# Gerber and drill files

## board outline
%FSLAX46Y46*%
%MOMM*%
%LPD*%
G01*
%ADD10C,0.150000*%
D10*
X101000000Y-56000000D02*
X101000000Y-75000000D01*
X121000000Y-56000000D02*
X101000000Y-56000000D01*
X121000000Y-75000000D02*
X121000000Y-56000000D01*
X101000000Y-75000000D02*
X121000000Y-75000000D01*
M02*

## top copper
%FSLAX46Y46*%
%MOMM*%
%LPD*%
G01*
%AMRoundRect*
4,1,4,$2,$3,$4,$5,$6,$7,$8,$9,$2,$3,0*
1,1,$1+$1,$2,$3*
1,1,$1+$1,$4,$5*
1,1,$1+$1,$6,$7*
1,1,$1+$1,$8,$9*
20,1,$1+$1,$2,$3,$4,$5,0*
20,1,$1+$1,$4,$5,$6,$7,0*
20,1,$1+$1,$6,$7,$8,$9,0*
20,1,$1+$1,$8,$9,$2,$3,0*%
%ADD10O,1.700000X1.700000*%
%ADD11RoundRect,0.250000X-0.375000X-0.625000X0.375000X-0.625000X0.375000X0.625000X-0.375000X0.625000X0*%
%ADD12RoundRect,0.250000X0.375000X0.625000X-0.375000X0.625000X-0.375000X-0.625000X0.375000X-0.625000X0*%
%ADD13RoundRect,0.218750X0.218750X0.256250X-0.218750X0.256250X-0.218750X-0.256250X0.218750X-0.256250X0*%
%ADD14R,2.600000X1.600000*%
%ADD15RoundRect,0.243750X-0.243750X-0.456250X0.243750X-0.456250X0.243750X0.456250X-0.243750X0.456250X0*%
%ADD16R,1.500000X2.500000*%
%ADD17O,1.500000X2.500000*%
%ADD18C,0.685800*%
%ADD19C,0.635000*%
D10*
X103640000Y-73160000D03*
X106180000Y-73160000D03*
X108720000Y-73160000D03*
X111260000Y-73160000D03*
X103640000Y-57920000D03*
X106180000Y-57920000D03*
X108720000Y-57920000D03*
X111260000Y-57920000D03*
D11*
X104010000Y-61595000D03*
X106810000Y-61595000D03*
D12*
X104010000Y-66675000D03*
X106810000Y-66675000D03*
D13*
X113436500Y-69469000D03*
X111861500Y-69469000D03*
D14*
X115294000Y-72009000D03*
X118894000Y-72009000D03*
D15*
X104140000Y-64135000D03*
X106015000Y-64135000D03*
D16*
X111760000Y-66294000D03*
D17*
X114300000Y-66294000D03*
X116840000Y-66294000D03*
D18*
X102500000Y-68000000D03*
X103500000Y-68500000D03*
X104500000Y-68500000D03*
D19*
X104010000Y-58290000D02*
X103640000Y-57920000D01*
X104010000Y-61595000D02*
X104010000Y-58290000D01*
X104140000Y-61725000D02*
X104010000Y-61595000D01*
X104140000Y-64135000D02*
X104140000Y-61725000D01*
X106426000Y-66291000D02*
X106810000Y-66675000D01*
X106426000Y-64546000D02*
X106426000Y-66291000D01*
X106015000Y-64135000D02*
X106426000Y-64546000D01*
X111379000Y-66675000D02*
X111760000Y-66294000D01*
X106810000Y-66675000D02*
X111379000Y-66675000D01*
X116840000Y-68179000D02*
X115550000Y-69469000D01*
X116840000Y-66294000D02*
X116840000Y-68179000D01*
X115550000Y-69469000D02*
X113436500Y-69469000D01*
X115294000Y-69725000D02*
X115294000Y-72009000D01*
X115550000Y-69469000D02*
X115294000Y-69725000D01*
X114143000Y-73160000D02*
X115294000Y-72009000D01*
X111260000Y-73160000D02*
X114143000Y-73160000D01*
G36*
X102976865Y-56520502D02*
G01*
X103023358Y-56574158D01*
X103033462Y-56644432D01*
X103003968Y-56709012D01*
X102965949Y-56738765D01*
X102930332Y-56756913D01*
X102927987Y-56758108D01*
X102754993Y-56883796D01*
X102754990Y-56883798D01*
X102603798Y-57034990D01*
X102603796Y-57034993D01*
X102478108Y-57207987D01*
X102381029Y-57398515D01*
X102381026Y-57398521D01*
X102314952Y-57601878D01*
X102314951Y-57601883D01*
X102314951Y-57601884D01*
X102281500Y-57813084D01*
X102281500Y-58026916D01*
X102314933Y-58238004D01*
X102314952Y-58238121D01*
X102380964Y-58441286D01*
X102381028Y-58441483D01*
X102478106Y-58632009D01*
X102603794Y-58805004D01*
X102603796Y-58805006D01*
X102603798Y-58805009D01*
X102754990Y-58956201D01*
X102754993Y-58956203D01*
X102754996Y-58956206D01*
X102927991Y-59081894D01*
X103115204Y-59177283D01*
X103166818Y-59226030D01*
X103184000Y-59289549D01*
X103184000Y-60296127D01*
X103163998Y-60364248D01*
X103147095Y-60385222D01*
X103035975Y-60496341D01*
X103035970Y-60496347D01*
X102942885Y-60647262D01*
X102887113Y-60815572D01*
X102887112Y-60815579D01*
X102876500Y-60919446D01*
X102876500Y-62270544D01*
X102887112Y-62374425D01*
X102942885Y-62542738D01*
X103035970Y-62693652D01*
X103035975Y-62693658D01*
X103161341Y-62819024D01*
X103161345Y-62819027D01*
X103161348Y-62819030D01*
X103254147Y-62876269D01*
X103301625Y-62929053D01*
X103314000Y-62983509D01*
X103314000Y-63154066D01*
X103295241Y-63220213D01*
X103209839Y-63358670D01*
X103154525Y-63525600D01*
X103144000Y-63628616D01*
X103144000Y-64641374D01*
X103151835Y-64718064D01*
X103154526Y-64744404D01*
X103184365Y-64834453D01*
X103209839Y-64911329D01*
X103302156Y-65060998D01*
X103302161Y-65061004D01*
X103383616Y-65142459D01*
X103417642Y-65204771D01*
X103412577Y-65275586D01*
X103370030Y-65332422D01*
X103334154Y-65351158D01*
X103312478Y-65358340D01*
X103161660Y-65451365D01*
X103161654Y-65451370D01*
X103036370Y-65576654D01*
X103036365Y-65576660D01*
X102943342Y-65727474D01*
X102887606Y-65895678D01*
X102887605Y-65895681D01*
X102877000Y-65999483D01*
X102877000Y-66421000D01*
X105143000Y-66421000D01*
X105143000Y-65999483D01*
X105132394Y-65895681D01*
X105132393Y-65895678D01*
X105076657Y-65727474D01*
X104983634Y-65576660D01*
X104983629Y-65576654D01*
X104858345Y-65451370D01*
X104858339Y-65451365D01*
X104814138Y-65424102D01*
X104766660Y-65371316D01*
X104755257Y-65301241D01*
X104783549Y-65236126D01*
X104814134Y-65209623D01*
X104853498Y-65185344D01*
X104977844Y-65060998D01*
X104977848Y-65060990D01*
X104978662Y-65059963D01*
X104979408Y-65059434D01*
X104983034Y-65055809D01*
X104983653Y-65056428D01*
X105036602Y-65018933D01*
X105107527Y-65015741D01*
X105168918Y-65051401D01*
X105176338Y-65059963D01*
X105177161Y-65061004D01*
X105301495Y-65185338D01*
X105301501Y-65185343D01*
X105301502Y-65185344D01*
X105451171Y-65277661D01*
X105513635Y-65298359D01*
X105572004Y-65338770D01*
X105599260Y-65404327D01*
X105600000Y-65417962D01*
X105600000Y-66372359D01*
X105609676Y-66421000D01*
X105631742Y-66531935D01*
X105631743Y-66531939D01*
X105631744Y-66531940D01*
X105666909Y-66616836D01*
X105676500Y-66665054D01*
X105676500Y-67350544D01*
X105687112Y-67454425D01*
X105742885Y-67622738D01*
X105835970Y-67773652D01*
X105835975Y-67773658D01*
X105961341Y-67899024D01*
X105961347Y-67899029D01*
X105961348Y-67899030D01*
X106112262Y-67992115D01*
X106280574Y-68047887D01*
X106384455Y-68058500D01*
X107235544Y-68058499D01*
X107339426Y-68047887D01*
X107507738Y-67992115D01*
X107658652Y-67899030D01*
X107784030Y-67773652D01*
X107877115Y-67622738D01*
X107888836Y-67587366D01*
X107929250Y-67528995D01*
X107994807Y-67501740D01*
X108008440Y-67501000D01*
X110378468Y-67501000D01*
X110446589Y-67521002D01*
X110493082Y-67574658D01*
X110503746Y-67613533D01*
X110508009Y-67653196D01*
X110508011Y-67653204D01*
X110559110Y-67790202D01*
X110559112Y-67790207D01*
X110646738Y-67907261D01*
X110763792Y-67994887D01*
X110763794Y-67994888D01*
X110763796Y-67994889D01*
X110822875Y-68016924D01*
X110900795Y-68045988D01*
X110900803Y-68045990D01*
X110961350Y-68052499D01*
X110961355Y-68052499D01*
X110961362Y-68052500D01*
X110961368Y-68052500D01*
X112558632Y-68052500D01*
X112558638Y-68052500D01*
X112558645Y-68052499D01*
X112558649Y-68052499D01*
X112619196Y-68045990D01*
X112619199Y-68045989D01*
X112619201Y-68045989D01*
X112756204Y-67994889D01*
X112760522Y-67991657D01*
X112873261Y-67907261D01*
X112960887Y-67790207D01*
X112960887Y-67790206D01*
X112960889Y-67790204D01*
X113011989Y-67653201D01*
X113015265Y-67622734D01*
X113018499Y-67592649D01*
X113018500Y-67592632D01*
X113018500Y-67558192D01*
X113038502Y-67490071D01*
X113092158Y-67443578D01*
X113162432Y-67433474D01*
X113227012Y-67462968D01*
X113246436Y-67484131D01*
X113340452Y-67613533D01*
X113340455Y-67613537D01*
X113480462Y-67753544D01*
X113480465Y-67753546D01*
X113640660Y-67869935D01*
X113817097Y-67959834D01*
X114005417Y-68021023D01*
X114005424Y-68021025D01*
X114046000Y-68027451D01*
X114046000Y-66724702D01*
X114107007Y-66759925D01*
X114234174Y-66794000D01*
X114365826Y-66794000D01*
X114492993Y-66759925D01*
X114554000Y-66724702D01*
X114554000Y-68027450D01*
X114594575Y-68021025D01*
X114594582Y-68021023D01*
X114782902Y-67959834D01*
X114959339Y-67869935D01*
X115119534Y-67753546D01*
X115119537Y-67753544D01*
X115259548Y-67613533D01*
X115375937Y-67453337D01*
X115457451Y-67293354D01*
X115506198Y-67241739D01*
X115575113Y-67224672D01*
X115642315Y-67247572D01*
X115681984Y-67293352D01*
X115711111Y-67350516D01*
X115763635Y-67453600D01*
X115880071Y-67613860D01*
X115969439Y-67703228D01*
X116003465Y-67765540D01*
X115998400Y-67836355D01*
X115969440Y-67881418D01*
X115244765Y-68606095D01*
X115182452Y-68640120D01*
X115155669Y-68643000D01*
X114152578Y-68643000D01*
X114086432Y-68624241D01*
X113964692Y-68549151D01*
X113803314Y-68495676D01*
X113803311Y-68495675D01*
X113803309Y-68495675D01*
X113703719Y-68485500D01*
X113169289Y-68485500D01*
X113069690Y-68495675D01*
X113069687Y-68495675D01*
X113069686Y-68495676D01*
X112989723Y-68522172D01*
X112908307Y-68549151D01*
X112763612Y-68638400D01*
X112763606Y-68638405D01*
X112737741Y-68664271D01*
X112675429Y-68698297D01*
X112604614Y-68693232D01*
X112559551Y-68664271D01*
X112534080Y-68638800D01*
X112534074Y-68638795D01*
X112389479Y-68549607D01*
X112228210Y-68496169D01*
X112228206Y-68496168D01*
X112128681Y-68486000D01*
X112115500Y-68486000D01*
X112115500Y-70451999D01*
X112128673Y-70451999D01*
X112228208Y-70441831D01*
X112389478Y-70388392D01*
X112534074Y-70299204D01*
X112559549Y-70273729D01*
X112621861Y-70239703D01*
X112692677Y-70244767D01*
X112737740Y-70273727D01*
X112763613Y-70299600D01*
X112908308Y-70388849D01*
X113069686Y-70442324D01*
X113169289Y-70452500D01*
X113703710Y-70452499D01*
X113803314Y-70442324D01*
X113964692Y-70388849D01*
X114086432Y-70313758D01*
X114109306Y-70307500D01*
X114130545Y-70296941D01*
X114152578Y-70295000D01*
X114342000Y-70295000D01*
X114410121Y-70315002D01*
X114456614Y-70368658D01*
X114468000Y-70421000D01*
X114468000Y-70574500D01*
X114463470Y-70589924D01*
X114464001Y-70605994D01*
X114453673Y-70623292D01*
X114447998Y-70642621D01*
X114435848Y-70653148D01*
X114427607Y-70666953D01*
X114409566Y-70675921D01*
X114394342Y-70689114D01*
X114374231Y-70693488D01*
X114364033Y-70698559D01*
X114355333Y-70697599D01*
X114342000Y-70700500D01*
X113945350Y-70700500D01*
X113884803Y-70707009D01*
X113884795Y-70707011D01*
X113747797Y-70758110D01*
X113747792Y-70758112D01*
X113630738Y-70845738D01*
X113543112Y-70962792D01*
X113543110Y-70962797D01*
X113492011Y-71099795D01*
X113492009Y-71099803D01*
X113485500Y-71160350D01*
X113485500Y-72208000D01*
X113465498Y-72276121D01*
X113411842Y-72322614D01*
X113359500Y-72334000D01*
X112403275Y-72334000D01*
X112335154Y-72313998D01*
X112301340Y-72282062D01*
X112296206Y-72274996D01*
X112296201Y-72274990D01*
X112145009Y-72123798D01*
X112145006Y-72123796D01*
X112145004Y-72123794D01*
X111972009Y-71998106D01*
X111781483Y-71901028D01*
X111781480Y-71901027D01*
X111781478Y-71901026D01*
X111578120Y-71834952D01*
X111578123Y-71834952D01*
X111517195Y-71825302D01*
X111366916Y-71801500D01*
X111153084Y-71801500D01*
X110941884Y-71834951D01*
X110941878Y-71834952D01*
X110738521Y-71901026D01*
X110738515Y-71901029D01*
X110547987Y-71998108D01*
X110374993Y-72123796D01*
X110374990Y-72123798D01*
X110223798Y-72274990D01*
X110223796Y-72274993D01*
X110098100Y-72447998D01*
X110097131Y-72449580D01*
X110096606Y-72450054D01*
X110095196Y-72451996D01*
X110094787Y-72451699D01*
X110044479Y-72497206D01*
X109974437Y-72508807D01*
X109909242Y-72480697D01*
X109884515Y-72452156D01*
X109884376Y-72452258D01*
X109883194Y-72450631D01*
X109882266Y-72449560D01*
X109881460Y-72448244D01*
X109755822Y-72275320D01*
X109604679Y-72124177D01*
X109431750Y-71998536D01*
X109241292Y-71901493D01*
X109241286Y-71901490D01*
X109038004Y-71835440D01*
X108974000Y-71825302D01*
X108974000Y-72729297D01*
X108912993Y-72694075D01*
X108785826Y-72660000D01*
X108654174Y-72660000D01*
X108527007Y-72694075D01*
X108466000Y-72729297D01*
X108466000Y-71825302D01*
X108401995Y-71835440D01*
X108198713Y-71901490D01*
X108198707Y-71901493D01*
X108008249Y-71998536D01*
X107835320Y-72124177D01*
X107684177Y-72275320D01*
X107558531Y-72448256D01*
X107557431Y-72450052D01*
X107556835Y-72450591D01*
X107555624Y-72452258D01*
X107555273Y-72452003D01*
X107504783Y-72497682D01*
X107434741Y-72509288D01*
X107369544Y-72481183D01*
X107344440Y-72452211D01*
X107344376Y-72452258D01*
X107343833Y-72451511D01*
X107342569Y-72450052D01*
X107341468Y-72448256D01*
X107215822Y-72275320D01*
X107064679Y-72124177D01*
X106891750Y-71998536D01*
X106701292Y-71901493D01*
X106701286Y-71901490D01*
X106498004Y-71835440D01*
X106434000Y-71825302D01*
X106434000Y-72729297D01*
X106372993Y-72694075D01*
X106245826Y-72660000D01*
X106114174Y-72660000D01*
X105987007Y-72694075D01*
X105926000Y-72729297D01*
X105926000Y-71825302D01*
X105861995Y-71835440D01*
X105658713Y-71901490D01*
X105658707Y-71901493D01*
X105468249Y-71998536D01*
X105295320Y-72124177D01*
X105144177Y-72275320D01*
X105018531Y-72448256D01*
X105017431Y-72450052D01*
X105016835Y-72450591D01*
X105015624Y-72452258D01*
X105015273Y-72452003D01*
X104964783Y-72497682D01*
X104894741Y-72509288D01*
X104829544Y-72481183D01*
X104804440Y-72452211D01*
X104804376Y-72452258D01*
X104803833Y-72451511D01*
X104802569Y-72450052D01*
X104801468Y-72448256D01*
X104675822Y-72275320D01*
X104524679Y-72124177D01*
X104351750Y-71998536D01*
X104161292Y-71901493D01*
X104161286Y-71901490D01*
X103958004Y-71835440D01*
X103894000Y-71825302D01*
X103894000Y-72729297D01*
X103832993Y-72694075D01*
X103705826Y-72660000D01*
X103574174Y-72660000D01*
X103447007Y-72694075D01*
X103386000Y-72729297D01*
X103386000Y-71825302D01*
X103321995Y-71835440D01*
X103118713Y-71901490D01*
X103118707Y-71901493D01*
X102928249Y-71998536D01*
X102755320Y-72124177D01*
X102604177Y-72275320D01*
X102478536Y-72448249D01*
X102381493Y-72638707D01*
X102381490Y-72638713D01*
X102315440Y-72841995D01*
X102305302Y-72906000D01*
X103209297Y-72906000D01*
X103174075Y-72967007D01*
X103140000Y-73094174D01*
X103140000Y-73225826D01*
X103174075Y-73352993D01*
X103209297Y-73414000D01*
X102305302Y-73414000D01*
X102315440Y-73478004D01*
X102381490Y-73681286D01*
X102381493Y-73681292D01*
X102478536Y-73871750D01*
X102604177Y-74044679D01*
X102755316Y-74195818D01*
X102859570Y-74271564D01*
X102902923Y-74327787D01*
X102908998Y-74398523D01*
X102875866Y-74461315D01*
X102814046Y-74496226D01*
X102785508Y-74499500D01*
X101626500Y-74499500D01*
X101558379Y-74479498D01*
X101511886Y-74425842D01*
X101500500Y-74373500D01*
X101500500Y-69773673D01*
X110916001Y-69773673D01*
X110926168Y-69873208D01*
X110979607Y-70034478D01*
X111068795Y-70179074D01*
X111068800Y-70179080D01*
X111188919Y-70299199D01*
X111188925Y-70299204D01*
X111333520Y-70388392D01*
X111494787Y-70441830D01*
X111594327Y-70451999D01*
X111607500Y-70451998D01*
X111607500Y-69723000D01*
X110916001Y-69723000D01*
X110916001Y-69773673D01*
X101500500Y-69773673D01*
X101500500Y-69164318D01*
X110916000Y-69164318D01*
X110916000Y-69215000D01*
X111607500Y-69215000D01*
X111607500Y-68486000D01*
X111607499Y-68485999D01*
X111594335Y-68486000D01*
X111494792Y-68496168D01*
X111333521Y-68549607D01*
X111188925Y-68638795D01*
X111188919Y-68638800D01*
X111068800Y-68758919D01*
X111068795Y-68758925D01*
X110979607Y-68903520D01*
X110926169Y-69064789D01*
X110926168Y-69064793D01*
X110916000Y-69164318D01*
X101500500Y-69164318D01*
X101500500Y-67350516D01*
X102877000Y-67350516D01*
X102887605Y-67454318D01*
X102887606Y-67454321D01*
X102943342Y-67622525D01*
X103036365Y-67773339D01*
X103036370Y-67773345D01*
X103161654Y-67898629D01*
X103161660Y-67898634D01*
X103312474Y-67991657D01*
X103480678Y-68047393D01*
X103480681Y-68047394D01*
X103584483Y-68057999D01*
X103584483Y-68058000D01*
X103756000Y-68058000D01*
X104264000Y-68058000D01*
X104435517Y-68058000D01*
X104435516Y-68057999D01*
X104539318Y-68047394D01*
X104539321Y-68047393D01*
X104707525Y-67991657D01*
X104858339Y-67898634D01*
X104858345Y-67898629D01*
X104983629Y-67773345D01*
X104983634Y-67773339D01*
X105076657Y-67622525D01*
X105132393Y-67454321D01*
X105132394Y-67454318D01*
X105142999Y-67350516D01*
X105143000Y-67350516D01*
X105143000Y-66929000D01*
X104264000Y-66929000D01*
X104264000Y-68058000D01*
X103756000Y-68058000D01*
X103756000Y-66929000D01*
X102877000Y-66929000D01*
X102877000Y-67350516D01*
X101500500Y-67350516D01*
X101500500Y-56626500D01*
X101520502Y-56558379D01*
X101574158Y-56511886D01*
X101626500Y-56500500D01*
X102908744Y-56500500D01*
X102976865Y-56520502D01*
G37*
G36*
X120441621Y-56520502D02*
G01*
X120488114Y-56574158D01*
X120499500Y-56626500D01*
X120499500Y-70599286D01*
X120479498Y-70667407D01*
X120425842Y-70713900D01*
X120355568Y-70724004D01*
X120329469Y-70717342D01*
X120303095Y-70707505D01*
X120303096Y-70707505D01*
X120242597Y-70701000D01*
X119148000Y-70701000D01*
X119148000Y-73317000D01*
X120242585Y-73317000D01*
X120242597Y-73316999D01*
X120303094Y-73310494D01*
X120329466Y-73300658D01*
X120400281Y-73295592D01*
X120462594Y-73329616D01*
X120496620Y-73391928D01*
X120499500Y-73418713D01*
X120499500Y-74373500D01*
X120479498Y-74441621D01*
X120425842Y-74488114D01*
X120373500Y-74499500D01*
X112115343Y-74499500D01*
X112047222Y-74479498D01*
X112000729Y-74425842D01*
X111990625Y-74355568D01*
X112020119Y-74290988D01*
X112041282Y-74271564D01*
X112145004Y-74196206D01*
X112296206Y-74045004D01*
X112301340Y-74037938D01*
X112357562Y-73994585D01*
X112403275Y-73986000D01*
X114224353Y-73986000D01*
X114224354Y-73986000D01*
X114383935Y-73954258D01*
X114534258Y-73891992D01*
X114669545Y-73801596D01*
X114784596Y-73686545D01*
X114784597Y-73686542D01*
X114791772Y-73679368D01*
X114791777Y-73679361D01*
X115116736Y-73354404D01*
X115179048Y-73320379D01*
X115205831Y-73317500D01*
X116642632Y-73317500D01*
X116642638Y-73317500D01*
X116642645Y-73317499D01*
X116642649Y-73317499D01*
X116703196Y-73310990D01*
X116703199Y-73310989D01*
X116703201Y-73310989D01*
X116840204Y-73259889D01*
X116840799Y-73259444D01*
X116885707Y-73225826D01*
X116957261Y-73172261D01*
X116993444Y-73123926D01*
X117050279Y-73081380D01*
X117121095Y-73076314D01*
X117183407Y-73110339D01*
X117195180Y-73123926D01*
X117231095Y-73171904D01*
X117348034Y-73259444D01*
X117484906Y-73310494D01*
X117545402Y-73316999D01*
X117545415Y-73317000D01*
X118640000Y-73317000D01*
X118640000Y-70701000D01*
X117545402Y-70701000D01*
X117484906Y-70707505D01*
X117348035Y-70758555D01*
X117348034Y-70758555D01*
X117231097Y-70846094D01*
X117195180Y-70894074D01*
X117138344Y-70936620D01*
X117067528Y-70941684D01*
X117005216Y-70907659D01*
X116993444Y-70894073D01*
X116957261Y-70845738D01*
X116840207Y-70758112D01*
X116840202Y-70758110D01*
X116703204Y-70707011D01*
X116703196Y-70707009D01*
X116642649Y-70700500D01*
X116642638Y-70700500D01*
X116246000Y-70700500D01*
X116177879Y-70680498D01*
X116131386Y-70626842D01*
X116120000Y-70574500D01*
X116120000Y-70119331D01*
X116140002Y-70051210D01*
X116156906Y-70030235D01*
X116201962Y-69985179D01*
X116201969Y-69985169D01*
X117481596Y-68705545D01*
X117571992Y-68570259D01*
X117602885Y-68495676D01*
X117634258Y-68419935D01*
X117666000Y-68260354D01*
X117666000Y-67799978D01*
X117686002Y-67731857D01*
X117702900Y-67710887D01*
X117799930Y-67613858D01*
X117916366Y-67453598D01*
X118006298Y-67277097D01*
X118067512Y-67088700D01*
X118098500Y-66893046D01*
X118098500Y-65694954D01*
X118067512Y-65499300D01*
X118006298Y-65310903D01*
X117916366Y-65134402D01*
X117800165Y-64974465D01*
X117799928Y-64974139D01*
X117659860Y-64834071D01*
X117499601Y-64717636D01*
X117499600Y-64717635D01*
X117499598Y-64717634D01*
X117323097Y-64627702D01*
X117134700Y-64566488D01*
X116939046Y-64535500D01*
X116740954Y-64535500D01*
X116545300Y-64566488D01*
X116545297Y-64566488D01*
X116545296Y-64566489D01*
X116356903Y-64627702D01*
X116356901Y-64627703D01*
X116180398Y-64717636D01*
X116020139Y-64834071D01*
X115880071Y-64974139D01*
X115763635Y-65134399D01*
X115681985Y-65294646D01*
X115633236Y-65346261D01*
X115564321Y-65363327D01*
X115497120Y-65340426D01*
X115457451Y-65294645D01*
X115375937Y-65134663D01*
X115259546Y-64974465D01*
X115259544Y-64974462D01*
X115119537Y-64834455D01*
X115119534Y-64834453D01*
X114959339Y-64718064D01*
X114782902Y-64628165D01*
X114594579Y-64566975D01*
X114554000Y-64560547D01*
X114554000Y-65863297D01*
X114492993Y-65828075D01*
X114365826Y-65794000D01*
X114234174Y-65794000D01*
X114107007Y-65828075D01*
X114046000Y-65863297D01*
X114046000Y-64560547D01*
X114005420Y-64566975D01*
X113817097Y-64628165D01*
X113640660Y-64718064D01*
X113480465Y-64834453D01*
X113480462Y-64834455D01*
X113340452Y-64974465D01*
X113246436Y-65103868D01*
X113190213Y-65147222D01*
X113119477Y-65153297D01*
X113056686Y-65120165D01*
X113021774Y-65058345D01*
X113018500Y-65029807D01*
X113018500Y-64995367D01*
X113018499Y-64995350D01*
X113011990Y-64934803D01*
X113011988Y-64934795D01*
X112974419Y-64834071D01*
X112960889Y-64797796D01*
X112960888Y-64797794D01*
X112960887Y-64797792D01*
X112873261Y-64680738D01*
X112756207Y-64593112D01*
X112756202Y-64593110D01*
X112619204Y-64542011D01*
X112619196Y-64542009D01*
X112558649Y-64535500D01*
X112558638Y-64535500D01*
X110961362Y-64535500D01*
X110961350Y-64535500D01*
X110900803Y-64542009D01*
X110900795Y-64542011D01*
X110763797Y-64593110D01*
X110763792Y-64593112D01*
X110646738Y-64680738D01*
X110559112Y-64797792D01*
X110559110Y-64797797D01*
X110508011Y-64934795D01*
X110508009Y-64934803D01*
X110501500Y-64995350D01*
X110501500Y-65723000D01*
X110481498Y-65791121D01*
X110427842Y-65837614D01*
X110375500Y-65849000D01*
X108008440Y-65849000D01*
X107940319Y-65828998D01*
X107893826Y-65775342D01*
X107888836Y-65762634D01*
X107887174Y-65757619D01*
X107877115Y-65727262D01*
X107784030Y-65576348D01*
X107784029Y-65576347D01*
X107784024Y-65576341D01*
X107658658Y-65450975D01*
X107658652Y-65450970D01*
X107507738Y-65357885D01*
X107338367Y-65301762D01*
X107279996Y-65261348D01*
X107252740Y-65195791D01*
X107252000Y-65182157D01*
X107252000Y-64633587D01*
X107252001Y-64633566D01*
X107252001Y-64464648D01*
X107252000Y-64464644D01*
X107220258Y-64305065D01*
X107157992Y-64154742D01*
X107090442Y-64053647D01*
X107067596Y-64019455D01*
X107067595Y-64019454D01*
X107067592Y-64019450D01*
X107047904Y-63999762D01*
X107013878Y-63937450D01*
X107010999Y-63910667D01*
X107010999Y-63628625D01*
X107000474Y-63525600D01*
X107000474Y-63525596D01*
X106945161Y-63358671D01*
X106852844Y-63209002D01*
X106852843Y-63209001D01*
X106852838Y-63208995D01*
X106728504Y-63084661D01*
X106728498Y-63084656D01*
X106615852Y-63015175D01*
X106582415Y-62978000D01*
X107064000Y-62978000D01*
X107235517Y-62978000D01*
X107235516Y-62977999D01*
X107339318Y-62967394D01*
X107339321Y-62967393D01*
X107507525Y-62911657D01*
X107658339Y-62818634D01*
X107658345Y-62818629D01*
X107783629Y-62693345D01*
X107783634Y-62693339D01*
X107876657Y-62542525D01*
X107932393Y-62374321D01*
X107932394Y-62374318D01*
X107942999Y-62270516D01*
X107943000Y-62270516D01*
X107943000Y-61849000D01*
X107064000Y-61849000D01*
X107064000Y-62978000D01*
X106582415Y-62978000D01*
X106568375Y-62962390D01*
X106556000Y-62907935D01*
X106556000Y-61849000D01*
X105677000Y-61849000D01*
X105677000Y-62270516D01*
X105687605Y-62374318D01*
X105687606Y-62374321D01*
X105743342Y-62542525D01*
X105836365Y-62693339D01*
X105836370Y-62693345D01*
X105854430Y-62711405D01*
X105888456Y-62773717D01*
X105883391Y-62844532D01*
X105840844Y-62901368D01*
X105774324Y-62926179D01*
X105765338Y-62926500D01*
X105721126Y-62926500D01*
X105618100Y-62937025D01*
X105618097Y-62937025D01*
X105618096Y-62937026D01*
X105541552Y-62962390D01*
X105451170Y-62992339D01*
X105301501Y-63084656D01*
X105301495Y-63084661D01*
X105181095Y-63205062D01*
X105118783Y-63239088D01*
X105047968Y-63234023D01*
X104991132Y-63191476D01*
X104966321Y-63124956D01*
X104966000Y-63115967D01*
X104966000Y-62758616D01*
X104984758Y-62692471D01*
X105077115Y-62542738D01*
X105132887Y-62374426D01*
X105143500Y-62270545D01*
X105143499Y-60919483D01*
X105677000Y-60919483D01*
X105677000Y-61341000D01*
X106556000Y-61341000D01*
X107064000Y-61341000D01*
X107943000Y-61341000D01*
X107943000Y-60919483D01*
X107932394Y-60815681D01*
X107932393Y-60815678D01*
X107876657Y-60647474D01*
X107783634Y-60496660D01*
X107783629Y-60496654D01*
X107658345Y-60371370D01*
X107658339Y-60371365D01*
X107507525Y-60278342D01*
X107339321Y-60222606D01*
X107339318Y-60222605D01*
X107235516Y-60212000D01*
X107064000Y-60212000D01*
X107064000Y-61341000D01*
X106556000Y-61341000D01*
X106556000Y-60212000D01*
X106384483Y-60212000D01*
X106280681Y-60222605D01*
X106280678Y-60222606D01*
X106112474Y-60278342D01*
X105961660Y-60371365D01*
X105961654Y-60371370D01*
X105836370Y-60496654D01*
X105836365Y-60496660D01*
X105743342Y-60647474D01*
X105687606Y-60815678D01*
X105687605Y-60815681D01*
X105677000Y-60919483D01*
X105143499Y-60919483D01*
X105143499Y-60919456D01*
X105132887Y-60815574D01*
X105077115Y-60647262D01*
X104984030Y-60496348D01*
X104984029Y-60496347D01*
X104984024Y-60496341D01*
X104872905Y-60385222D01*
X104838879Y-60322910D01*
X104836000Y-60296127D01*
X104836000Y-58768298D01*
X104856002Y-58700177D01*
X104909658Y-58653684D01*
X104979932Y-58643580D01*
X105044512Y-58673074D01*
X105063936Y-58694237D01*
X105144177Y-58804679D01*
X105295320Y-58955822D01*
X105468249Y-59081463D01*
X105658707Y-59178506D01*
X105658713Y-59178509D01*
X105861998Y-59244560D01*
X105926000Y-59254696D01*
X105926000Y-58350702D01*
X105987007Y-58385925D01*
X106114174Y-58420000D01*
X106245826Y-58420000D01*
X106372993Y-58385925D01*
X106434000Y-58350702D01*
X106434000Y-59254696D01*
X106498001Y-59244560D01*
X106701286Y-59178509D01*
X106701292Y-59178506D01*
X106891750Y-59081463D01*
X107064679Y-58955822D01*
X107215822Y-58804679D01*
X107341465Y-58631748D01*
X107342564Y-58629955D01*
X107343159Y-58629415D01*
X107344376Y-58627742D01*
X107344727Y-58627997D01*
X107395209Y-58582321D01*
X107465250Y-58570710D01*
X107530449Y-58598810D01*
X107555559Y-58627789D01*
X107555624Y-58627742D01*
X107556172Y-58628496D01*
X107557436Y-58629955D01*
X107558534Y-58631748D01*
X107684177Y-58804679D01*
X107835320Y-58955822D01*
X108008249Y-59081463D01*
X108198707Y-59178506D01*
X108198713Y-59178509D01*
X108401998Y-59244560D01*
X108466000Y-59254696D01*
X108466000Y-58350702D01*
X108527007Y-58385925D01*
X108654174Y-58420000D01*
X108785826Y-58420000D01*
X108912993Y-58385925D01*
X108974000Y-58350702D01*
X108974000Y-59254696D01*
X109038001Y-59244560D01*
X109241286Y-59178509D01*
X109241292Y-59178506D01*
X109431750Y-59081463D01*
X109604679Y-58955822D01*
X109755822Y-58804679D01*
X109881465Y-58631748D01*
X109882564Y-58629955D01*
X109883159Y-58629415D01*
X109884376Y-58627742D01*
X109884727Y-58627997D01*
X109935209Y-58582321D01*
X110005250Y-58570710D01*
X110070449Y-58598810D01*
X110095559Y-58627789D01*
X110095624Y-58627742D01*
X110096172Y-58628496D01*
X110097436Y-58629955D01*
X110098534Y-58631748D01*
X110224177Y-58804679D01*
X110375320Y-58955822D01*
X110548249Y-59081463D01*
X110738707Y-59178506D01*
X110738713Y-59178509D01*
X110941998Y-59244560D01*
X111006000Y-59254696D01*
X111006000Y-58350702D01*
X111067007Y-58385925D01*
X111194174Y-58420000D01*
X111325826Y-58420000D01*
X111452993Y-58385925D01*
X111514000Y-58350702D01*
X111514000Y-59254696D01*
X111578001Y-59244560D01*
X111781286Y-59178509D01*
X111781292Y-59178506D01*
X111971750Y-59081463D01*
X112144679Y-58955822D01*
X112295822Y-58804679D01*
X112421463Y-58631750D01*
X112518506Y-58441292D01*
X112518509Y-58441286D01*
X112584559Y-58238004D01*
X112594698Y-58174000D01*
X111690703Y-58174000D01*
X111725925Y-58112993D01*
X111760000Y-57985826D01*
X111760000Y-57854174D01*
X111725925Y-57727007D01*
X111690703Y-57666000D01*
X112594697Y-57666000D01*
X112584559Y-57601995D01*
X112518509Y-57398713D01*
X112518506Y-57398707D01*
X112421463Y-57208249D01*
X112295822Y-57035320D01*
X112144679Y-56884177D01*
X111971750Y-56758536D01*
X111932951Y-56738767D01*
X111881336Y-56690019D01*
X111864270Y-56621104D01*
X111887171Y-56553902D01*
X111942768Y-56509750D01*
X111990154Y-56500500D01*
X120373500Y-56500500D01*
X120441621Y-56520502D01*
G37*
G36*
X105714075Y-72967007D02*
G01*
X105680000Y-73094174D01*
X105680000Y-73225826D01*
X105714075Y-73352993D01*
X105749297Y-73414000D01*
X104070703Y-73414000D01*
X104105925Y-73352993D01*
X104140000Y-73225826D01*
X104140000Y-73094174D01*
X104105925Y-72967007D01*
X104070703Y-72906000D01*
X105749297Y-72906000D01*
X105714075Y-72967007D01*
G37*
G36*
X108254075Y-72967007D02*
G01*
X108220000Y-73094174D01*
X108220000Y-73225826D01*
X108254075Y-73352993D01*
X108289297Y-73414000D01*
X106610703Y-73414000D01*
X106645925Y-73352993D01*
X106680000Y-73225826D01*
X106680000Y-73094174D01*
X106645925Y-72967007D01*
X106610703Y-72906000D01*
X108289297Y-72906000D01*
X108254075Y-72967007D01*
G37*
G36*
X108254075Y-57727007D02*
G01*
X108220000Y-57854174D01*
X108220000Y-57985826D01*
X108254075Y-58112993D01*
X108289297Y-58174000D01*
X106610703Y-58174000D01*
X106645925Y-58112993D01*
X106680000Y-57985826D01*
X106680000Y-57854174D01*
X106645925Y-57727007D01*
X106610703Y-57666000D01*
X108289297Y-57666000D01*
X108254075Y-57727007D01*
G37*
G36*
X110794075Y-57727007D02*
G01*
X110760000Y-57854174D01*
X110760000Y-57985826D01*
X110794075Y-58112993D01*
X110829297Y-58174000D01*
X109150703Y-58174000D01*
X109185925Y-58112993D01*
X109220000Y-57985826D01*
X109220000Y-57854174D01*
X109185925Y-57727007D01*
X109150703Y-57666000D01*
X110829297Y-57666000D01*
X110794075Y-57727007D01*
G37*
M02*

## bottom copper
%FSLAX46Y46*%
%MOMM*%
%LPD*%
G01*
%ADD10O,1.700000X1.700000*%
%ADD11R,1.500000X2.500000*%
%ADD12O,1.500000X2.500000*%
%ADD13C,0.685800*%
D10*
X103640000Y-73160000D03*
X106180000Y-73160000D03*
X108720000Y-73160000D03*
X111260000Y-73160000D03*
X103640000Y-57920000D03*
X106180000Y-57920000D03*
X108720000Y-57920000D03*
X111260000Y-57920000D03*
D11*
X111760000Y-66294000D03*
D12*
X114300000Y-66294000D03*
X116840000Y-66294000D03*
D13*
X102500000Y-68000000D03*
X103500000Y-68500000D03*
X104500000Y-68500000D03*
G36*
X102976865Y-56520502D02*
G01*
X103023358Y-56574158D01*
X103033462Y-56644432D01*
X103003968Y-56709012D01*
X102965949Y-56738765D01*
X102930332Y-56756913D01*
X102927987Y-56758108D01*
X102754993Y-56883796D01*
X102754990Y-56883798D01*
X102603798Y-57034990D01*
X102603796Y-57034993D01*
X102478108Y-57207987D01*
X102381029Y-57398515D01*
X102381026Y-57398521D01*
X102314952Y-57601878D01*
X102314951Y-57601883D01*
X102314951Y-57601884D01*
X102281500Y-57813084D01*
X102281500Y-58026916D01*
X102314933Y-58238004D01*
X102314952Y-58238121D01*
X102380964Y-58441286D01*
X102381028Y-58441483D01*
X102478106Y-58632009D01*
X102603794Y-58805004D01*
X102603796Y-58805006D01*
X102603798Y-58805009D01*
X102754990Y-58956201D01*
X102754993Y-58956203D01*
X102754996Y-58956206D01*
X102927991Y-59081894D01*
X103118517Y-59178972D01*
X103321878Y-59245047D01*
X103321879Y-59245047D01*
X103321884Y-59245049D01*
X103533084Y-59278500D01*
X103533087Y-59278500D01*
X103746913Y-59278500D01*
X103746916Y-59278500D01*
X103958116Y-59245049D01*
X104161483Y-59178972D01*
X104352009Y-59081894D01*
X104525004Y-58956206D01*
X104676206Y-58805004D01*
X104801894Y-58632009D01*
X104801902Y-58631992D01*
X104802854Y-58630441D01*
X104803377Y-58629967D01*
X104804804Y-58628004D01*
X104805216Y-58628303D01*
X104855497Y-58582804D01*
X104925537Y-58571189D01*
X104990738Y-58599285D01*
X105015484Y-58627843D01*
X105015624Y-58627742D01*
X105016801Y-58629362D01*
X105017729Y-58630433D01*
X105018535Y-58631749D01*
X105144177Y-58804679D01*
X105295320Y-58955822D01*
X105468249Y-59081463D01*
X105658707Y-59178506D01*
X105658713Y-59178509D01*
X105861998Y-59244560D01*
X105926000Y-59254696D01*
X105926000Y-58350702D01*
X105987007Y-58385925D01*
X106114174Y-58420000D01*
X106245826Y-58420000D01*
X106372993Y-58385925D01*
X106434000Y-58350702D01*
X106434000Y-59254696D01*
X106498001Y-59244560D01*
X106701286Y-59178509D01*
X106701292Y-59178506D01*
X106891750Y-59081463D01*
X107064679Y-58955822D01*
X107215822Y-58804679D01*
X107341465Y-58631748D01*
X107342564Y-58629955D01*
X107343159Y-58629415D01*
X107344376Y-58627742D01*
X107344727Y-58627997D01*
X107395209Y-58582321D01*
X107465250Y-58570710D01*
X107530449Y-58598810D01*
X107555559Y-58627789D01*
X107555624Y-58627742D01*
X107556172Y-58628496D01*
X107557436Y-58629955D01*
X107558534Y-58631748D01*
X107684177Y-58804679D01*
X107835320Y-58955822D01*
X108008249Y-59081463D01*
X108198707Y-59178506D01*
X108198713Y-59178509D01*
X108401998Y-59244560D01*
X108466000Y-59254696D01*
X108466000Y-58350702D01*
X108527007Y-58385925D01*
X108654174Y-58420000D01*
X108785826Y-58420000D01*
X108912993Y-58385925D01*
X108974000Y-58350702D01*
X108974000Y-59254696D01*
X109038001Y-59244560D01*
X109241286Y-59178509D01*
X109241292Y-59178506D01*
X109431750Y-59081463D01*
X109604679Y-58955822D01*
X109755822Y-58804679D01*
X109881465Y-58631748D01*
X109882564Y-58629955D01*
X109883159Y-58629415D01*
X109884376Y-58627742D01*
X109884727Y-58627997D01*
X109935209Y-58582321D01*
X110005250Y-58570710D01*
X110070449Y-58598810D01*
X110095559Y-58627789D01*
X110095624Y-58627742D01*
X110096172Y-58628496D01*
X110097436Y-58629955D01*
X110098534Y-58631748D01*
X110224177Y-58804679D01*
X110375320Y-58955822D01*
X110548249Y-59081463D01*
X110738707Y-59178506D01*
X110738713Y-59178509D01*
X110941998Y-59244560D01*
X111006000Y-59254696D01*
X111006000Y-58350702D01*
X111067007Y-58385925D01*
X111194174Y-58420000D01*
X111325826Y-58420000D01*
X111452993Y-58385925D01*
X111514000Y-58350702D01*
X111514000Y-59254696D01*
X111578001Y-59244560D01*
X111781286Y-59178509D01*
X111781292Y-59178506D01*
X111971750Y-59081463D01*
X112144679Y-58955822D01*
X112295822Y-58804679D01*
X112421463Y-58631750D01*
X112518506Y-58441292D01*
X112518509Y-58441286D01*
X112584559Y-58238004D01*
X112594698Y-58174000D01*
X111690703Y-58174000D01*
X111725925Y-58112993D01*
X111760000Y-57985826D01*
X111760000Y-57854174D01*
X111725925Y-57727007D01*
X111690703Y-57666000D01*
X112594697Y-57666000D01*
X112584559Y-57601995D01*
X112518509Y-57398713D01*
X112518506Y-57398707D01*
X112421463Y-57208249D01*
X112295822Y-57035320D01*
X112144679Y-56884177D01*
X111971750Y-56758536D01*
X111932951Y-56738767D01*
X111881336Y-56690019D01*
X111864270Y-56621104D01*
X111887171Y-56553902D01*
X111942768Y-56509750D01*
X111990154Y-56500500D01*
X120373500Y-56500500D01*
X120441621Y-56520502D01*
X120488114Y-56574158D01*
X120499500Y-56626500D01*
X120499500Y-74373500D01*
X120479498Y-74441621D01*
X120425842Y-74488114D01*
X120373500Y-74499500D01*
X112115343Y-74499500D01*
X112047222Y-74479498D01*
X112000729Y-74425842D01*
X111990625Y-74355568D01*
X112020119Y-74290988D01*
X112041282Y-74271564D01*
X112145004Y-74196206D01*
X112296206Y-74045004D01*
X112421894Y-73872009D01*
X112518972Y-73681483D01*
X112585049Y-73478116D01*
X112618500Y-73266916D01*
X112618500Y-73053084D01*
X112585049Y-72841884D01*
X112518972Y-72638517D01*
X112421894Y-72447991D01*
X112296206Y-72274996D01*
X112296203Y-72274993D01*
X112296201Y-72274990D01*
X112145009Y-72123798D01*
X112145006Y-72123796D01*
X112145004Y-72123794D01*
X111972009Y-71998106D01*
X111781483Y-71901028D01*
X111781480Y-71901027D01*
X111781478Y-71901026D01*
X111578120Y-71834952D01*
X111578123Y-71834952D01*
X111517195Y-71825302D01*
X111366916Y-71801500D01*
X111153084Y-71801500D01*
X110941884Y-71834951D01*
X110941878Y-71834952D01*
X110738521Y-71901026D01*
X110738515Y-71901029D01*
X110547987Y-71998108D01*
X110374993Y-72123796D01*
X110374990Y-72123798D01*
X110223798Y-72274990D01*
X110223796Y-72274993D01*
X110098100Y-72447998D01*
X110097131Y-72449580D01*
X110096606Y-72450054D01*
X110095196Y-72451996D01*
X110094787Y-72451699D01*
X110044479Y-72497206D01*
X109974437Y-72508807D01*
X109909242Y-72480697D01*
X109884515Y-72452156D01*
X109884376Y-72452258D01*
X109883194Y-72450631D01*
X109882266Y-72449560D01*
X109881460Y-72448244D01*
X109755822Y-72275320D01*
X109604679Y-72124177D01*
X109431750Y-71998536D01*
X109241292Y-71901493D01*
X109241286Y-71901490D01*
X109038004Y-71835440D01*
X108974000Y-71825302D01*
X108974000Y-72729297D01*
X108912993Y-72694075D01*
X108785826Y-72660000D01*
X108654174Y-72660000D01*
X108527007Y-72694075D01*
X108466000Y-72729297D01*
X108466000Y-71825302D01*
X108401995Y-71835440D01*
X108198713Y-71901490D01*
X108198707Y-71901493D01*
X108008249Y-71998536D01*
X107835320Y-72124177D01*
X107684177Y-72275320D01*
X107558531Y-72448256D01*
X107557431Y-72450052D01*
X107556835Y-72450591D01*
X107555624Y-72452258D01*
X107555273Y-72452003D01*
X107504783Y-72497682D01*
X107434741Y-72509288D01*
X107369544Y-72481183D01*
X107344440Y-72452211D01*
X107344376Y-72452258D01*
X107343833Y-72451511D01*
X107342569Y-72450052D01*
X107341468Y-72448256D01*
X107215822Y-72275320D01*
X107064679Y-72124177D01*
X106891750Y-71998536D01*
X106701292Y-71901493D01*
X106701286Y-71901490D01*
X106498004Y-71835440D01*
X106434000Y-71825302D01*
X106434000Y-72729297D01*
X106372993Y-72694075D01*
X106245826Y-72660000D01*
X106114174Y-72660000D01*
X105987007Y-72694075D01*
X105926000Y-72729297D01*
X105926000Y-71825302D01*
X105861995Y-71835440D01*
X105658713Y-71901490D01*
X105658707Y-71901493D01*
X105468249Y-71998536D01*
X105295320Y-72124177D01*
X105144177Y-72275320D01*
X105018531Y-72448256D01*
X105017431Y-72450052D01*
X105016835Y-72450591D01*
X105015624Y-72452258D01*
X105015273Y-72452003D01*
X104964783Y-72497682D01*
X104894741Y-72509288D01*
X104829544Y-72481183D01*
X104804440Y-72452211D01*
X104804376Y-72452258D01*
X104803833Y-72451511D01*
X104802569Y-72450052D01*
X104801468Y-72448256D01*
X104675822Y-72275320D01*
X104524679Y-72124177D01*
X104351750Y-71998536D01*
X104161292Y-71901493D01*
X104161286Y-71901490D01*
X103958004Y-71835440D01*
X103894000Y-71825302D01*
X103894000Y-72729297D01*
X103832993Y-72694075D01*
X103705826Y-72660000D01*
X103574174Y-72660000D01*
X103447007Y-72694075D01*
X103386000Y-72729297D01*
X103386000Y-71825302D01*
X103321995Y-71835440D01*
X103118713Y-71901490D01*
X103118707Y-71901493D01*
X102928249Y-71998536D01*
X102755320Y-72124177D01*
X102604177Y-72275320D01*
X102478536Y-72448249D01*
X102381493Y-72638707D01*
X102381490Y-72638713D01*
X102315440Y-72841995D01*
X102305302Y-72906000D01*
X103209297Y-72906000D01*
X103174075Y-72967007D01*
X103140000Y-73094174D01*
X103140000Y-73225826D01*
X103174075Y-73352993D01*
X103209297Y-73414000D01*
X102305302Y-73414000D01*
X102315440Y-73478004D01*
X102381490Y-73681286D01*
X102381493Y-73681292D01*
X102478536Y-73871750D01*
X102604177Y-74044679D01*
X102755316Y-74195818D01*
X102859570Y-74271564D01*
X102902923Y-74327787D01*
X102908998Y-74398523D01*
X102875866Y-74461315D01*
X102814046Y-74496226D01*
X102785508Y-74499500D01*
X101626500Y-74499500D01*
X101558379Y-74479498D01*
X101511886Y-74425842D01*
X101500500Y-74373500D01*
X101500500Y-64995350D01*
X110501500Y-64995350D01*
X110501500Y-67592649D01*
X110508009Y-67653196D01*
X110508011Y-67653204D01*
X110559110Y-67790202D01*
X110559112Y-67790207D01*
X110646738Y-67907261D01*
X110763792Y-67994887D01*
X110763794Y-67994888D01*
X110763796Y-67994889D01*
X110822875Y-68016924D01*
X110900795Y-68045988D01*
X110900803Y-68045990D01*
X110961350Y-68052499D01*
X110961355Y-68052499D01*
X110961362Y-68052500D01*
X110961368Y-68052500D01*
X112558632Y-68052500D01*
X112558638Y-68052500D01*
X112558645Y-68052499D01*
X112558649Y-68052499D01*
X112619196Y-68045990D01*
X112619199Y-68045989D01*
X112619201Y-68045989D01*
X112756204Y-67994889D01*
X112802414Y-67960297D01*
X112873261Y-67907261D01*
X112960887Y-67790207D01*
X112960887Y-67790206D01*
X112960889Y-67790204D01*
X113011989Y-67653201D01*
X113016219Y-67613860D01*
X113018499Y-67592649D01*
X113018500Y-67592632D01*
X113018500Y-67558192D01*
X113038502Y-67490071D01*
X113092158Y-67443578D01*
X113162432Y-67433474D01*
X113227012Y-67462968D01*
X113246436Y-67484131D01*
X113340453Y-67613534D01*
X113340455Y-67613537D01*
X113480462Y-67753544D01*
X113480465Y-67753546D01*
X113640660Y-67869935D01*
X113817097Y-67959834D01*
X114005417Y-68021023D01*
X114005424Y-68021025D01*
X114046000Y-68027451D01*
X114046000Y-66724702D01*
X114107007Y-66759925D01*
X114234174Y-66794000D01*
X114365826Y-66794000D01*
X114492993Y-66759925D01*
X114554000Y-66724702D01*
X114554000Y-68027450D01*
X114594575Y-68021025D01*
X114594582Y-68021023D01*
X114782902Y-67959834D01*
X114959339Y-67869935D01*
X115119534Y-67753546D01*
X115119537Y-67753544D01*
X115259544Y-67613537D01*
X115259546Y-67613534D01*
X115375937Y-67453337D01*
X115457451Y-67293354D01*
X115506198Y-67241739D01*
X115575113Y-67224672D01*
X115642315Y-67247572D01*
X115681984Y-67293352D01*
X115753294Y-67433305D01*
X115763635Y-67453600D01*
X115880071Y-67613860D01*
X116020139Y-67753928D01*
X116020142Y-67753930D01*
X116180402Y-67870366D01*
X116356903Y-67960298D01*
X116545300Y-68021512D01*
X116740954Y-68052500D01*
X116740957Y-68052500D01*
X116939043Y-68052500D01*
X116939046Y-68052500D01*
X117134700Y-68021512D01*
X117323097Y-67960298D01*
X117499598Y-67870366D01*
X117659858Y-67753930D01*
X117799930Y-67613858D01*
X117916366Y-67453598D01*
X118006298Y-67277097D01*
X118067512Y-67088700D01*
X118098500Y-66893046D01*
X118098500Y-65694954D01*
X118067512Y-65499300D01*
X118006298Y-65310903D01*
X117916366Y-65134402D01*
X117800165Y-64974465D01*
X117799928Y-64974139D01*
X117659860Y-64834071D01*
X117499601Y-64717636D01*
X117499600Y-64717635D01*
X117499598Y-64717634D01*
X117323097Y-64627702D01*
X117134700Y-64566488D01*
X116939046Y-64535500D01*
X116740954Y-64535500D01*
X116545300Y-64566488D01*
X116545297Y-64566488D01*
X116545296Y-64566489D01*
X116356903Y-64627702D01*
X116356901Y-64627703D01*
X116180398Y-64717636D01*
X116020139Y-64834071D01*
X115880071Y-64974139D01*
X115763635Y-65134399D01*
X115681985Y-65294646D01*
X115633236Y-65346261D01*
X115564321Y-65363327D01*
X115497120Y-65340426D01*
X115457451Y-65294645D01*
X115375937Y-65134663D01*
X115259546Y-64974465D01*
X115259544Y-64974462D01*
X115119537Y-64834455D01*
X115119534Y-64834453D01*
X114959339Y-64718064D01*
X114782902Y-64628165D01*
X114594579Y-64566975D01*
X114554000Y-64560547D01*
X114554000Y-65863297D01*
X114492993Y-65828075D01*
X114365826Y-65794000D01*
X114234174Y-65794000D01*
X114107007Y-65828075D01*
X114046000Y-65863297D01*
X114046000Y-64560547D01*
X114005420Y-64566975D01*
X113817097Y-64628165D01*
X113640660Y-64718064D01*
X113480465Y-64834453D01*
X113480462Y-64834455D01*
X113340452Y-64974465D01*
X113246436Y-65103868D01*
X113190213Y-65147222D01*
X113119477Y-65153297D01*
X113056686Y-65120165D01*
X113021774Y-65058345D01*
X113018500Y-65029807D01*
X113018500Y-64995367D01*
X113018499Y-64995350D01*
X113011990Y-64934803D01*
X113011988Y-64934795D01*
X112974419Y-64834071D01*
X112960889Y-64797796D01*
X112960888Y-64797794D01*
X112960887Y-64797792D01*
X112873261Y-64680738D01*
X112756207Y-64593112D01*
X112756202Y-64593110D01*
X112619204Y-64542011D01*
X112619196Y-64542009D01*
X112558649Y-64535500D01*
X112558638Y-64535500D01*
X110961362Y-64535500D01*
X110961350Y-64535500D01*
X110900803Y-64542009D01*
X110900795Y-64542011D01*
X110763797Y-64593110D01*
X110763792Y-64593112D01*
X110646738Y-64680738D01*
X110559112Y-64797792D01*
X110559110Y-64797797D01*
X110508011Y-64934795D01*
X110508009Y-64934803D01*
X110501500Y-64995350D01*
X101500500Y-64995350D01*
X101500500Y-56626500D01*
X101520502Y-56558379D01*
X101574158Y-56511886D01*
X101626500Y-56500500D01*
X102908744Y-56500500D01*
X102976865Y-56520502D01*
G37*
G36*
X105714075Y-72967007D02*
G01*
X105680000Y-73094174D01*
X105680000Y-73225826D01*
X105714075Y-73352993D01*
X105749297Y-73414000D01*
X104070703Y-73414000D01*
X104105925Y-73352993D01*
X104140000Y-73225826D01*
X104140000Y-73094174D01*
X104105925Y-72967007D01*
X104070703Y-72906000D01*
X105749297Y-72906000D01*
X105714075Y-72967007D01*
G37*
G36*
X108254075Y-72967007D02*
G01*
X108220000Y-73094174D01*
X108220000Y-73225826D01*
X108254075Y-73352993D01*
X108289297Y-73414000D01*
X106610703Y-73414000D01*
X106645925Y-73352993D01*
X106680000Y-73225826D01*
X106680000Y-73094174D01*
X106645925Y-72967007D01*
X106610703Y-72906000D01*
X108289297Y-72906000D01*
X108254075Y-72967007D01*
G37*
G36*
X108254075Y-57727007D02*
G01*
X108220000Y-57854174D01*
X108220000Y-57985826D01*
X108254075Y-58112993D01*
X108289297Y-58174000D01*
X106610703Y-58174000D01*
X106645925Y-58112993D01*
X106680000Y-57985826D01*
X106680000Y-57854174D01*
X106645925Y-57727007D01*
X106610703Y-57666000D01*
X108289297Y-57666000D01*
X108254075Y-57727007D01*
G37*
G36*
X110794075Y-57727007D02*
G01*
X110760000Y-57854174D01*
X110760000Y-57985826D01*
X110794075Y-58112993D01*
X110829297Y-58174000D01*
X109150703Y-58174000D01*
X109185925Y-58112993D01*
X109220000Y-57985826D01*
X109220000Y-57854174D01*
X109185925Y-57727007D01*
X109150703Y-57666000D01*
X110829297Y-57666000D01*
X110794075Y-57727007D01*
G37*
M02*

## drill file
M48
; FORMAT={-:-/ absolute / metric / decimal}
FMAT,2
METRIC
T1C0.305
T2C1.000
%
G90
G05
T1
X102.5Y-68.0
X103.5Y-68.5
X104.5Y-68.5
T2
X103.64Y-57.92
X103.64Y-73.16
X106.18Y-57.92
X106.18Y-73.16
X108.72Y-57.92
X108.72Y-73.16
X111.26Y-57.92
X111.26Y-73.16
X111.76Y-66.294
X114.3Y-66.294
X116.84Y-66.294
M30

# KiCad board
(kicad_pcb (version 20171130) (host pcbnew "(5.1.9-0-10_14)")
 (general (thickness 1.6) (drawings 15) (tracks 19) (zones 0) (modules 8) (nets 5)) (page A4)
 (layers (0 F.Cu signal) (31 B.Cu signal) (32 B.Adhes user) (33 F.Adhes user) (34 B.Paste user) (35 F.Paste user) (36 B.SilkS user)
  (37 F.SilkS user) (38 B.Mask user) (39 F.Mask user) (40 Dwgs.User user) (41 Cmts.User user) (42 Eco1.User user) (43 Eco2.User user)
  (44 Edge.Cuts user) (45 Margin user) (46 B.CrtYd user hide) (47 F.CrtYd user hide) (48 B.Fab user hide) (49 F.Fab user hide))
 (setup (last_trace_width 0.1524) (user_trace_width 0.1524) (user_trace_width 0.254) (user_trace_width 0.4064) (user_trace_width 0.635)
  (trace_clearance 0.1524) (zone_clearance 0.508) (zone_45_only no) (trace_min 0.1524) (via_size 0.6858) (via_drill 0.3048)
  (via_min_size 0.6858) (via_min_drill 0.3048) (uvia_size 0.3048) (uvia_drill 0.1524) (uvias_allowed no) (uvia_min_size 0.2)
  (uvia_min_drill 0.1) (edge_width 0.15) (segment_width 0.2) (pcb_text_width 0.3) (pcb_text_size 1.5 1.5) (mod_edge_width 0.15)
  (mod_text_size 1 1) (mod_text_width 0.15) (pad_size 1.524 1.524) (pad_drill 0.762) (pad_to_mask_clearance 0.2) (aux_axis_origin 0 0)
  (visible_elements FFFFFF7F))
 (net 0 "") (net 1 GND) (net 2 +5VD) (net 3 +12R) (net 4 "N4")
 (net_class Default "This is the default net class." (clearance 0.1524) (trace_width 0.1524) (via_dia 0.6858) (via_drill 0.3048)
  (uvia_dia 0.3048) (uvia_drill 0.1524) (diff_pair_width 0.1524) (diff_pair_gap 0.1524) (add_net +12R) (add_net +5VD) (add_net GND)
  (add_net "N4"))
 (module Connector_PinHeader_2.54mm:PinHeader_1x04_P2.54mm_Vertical (layer B.Cu) (at 111.26 73.16 90)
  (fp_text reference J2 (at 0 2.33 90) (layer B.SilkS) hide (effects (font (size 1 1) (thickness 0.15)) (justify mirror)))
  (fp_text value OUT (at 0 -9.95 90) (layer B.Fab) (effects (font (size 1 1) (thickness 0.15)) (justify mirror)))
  (pad 4 thru_hole oval (at 0 -7.62 90) (size 1.7 1.7) (drill 1) (layers *.Cu *.Mask) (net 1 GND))
  (pad 3 thru_hole oval (at 0 -5.08 90) (size 1.7 1.7) (drill 1) (layers *.Cu *.Mask) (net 1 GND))
  (pad 2 thru_hole oval (at 0 -2.54 90) (size 1.7 1.7) (drill 1) (layers *.Cu *.Mask) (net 1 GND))
  (pad 1 thru_hole oval (at 0 0 90) (size 1.7 1.7) (drill 1) (layers *.Cu *.Mask) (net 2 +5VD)))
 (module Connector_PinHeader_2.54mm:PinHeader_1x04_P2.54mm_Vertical (layer B.Cu) (at 103.64 57.92 270)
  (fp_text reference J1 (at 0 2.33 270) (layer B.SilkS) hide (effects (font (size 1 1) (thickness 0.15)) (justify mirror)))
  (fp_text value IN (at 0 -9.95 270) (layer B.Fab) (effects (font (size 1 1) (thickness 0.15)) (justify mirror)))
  (pad 1 thru_hole oval (at 0 0 270) (size 1.7 1.7) (drill 1) (layers *.Cu *.Mask) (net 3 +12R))
  (pad 2 thru_hole oval (at 0 -2.54 270) (size 1.7 1.7) (drill 1) (layers *.Cu *.Mask) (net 1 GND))
  (pad 3 thru_hole oval (at 0 -5.08 270) (size 1.7 1.7) (drill 1) (layers *.Cu *.Mask) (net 1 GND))
  (pad 4 thru_hole oval (at 0 -7.62 270) (size 1.7 1.7) (drill 1) (layers *.Cu *.Mask) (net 1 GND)))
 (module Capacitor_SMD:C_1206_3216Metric (layer F.Cu) (at 105.41 61.595)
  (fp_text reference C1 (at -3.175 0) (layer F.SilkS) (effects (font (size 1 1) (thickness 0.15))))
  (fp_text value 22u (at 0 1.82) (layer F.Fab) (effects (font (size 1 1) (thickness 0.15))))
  (pad 1 smd roundrect (at -1.4 0) (size 1.25 1.75) (layers F.Cu F.Paste F.Mask) (roundrect_rratio 0.2) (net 3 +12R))
  (pad 2 smd roundrect (at 1.4 0) (size 1.25 1.75) (layers F.Cu F.Paste F.Mask) (roundrect_rratio 0.2) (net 1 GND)))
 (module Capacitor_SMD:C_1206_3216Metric (layer F.Cu) (at 105.41 66.675 180)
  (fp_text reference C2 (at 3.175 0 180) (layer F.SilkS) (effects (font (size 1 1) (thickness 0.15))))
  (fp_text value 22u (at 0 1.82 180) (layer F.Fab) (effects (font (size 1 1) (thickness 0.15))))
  (pad 2 smd roundrect (at 1.4 0 180) (size 1.25 1.75) (layers F.Cu F.Paste F.Mask) (roundrect_rratio 0.2) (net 1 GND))
  (pad 1 smd roundrect (at -1.4 0 180) (size 1.25 1.75) (layers F.Cu F.Paste F.Mask) (roundrect_rratio 0.2) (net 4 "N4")))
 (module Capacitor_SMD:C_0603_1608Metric (layer F.Cu) (at 112.649 69.469 180)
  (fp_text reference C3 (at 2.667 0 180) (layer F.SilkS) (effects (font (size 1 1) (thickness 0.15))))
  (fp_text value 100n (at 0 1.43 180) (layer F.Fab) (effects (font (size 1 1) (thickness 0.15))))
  (pad 1 smd roundrect (at -0.7875 0 180) (size 0.875 0.95) (layers F.Cu F.Paste F.Mask) (roundrect_rratio 0.25) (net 2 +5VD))
  (pad 2 smd roundrect (at 0.7875 0 180) (size 0.875 0.95) (layers F.Cu F.Paste F.Mask) (roundrect_rratio 0.25) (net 1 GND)))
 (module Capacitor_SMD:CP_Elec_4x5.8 (layer F.Cu) (at 117.094 72.009)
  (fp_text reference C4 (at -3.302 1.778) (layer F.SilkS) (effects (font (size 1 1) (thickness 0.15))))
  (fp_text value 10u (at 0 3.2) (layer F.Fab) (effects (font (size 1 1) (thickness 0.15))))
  (pad 1 smd rect (at -1.8 0) (size 2.6 1.6) (layers F.Cu F.Paste F.Mask) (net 2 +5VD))
  (pad 2 smd rect (at 1.8 0) (size 2.6 1.6) (layers F.Cu F.Paste F.Mask) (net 1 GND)))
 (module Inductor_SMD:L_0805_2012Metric (layer F.Cu) (at 105.0775 64.135)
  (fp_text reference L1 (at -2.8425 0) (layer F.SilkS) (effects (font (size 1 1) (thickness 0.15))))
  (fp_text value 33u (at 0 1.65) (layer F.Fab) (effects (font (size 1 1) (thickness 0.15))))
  (pad 1 smd roundrect (at -0.9375 0) (size 0.975 1.4) (layers F.Cu F.Paste F.Mask) (roundrect_rratio 0.25) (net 3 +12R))
  (pad 2 smd roundrect (at 0.9375 0) (size 0.975 1.4) (layers F.Cu F.Paste F.Mask) (roundrect_rratio 0.25) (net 4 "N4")))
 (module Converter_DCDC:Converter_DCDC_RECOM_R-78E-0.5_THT (layer F.Cu) (at 111.76 66.294)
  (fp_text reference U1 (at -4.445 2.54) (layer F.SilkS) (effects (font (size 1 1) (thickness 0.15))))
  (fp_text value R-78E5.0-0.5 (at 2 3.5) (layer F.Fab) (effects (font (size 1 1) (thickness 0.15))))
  (pad 1 thru_hole rect (at 0 0) (size 1.5 2.5) (drill 1) (layers *.Cu *.Mask) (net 4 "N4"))
  (pad 2 thru_hole oval (at 2.54 0) (size 1.5 2.5) (drill 1) (layers *.Cu *.Mask) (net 1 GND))
  (pad 3 thru_hole oval (at 5.08 0) (size 1.5 2.5) (drill 1) (layers *.Cu *.Mask) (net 2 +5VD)))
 (gr_line (start 101 56) (end 101 75) (layer Edge.Cuts) (width 0.15))
 (gr_line (start 121 56) (end 101 56) (layer Edge.Cuts) (width 0.15))
 (gr_line (start 121 75) (end 121 56) (layer Edge.Cuts) (width 0.15))
 (gr_line (start 101 75) (end 121 75) (layer Edge.Cuts) (width 0.15))
 (via (at 102.5 68) (size 0.6858) (drill 0.3048) (layers F.Cu B.Cu) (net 1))
 (via (at 103.5 68.5) (size 0.6858) (drill 0.3048) (layers F.Cu B.Cu) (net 1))
 (via (at 104.5 68.5) (size 0.6858) (drill 0.3048) (layers F.Cu B.Cu) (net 1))
 (segment (start 104.01 58.29) (end 103.64 57.92) (width 0.635) (layer F.Cu) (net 3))
 (segment (start 104.01 61.595) (end 104.01 58.29) (width 0.635) (layer F.Cu) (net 3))
 (segment (start 104.14 61.725) (end 104.01 61.595) (width 0.635) (layer F.Cu) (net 3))
 (segment (start 104.14 64.135) (end 104.14 61.725) (width 0.635) (layer F.Cu) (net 3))
 (segment (start 106.426 66.291) (end 106.81 66.675) (width 0.635) (layer F.Cu) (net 4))
 (segment (start 106.426 64.546) (end 106.426 66.291) (width 0.635) (layer F.Cu) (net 4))
 (segment (start 106.015 64.135) (end 106.426 64.546) (width 0.635) (layer F.Cu) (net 4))
 (segment (start 111.379 66.675) (end 111.76 66.294) (width 0.635) (layer F.Cu) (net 4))
 (segment (start 106.81 66.675) (end 111.379 66.675) (width 0.635) (layer F.Cu) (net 4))
 (segment (start 116.84 68.179) (end 115.55 69.469) (width 0.635) (layer F.Cu) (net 2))
 (segment (start 116.84 66.294) (end 116.84 68.179) (width 0.635) (layer F.Cu) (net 2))
 (segment (start 115.55 69.469) (end 113.4365 69.469) (width 0.635) (layer F.Cu) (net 2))
 (segment (start 115.294 69.725) (end 115.294 72.009) (width 0.635) (layer F.Cu) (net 2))
 (segment (start 115.55 69.469) (end 115.294 69.725) (width 0.635) (layer F.Cu) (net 2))
 (segment (start 114.143 73.16) (end 115.294 72.009) (width 0.635) (layer F.Cu) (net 2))
 (segment (start 111.26 73.16) (end 114.143 73.16) (width 0.635) (layer F.Cu) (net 2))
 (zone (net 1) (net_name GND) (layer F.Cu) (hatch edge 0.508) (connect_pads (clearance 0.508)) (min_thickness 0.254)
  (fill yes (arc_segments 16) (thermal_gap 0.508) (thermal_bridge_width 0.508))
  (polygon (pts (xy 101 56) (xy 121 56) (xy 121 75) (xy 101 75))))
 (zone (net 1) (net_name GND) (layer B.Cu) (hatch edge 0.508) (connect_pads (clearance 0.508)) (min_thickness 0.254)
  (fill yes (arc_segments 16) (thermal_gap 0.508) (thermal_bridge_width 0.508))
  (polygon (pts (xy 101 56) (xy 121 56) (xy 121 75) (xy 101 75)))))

